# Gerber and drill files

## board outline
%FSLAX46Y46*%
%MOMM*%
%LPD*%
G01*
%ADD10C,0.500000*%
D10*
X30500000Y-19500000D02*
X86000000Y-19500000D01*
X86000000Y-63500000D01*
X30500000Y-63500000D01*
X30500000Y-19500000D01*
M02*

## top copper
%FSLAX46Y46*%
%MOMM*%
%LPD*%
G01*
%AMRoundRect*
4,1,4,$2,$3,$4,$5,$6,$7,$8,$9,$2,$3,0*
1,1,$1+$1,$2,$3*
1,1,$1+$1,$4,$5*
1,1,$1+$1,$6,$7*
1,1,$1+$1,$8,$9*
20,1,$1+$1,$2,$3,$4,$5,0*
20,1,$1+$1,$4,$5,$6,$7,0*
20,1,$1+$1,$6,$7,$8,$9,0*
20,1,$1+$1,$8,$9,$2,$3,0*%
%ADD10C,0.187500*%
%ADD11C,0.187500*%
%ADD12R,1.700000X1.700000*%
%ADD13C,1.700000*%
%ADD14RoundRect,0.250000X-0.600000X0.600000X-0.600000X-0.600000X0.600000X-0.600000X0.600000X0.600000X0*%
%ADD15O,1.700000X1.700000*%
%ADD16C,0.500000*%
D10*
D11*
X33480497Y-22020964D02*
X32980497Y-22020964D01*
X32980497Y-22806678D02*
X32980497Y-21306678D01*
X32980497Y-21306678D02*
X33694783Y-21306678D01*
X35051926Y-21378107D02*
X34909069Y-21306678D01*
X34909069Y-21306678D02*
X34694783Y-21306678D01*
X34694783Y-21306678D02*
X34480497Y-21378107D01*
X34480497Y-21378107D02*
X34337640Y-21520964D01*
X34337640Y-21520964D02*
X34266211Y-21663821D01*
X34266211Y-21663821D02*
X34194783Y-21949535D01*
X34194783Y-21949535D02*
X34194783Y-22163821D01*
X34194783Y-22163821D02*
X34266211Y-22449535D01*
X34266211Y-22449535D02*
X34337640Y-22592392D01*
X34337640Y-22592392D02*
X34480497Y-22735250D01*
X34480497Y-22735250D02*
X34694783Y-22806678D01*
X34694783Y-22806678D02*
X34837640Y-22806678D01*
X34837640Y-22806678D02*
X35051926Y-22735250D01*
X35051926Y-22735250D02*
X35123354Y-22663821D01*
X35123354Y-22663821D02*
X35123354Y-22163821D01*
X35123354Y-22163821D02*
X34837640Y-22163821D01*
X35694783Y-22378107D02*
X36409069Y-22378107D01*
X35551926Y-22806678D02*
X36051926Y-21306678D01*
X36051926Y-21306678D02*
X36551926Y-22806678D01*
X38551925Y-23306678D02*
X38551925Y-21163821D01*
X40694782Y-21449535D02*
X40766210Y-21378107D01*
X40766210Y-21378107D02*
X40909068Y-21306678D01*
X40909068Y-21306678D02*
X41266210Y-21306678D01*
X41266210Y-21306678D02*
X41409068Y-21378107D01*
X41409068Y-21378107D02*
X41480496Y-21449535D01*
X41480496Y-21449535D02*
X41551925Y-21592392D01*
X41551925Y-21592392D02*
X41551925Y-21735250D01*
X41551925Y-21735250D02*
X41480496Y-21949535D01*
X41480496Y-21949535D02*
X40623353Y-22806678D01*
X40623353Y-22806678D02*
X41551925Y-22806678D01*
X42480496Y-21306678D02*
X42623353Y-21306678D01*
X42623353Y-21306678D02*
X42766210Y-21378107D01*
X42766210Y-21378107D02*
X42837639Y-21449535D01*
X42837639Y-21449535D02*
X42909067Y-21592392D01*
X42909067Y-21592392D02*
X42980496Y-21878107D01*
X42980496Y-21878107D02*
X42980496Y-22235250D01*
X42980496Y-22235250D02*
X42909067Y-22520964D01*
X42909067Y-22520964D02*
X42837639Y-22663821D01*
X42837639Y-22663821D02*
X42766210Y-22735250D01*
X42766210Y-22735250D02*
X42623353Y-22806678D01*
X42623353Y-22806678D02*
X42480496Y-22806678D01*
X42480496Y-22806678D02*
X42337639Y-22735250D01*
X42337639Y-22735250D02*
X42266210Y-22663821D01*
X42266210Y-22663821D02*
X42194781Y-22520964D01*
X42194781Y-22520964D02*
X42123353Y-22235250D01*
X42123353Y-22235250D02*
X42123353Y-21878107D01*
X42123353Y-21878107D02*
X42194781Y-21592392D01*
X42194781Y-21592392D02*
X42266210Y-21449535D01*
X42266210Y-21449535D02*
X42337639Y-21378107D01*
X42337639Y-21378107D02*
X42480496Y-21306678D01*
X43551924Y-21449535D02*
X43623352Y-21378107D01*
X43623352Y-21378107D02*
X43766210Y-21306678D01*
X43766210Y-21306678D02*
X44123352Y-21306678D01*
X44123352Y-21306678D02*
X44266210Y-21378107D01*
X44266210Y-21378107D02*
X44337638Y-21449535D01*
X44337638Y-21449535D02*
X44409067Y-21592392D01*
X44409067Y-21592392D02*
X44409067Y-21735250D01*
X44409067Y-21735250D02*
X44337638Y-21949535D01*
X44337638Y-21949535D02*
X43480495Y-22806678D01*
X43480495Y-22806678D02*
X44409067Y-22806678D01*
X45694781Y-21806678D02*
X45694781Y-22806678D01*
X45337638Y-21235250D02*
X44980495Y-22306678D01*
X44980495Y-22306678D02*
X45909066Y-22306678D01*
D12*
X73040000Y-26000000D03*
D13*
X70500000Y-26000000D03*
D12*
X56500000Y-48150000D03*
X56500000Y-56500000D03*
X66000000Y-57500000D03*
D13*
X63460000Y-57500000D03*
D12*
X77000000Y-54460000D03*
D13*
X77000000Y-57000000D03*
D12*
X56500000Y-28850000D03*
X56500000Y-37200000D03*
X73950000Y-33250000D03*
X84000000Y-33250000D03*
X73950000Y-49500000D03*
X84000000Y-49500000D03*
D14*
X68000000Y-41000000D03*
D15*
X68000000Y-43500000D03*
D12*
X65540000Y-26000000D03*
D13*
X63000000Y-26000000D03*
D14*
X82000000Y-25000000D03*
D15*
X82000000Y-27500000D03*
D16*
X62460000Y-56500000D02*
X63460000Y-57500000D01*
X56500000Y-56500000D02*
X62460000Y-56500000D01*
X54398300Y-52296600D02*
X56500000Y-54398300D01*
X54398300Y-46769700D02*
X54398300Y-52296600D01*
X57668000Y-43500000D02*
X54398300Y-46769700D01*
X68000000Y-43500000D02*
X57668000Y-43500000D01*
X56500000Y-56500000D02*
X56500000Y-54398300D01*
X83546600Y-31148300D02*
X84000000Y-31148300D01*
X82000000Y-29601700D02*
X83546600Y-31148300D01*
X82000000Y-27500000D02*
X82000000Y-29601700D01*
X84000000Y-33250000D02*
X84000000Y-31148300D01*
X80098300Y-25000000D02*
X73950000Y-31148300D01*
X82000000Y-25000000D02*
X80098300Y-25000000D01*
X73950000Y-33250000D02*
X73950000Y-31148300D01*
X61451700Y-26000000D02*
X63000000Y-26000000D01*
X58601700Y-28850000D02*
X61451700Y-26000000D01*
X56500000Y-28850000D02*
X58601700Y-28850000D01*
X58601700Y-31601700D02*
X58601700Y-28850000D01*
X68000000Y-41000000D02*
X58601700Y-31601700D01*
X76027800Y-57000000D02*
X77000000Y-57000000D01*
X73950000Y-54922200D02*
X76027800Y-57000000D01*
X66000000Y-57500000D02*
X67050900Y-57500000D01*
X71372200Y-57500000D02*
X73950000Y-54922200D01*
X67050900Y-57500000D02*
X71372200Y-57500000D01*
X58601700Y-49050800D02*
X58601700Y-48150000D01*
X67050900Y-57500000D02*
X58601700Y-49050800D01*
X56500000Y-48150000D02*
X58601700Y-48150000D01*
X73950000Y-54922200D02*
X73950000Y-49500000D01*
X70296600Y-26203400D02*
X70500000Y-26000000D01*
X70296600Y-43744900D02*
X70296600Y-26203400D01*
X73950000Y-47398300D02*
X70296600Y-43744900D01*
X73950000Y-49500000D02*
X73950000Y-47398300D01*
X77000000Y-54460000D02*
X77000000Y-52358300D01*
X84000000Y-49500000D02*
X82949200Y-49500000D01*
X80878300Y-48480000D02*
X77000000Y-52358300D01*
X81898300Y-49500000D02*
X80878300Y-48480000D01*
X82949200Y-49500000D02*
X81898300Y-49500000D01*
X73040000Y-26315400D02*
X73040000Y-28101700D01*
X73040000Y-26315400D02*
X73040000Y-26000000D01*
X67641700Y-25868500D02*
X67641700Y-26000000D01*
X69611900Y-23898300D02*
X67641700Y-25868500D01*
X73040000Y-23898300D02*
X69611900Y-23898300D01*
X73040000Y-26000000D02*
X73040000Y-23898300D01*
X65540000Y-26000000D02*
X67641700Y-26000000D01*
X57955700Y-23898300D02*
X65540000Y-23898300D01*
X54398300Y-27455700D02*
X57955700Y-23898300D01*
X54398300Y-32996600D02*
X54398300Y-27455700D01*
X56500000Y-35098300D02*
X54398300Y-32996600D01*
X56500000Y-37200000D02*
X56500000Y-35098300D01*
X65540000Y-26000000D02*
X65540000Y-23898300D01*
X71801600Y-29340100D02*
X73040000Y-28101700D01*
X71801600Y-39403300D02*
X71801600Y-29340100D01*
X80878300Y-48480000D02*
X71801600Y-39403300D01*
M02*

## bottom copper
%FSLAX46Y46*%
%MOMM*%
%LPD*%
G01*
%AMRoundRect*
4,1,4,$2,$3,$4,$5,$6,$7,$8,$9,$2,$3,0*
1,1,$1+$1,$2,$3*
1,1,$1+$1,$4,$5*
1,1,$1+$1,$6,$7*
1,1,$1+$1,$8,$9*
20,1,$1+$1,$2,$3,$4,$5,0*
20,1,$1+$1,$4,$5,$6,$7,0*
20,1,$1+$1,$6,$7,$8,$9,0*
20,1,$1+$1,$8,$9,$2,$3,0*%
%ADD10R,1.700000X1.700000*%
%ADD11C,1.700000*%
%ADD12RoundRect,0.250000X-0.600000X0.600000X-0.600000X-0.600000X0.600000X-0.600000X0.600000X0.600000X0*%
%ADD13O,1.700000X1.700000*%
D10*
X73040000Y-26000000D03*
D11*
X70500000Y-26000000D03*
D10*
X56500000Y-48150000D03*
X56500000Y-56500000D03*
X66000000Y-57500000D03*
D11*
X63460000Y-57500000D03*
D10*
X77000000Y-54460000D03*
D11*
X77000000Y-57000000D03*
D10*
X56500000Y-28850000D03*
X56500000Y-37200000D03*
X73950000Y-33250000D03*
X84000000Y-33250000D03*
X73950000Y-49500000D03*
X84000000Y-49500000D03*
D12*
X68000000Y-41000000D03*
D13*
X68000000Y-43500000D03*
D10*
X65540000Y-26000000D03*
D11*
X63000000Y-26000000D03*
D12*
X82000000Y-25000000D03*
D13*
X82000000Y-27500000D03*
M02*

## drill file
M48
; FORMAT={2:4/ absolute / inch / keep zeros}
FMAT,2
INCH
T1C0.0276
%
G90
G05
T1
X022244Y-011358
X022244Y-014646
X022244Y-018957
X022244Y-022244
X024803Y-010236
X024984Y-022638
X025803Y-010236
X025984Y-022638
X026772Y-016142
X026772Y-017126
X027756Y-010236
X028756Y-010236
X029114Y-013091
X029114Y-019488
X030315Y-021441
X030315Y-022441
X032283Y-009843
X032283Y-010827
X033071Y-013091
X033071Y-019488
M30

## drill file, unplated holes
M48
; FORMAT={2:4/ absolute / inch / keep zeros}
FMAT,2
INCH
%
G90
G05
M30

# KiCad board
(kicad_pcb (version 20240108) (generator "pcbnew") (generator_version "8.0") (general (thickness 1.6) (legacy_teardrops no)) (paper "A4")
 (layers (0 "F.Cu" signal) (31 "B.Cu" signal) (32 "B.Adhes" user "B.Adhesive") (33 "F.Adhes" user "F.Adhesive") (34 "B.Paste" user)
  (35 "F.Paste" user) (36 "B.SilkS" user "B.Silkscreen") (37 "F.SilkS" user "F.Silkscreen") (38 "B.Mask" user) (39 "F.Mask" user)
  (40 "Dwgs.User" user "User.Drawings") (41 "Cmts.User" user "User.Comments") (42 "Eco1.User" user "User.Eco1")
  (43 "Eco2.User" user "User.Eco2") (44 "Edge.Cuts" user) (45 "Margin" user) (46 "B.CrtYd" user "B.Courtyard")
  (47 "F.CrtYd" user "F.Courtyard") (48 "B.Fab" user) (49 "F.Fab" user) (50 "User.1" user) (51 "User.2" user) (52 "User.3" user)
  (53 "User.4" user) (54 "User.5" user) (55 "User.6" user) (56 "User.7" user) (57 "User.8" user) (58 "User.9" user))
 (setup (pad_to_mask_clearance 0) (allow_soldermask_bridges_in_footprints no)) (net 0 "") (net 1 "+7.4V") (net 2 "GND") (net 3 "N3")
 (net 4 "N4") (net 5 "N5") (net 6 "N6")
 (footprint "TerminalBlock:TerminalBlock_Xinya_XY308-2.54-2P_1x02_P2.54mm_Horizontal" (layer "F.Cu") (at 73.04 26 180)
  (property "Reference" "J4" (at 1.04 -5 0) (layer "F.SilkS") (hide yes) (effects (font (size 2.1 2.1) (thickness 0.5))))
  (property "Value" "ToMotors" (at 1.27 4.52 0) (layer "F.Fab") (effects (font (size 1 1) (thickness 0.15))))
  (pad "1" thru_hole rect (at 0 0 180) (size 1.7 1.7) (drill 0.7) (layers "*.Cu" "*.Mask") (remove_unused_layers no) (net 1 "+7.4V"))
  (pad "2" thru_hole circle (at 2.54 0 180) (size 1.7 1.7) (drill 0.7) (layers "*.Cu" "*.Mask") (remove_unused_layers no) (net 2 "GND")))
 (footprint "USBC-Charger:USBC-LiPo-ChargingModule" (layer "F.Cu") (at 45.5 61.6)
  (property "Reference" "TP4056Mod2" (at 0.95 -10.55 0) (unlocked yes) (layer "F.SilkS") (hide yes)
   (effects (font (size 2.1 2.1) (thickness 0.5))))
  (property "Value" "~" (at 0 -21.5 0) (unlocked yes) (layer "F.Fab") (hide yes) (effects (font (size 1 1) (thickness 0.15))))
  (pad "1" thru_hole rect (at 11 -13.45) (size 1.7 1.7) (drill 0.7) (layers "*.Cu" "*.Mask") (remove_unused_layers no) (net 2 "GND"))
  (pad "2" thru_hole rect (at 11 -5.1) (size 1.7 1.7) (drill 0.7) (layers "*.Cu" "*.Mask") (remove_unused_layers no) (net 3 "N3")))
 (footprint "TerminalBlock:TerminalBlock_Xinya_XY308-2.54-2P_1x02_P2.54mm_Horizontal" (layer "F.Cu") (at 66 57.5 180)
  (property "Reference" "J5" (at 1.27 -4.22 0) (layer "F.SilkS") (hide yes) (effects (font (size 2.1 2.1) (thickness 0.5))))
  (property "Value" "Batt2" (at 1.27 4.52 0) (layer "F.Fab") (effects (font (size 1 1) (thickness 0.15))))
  (pad "1" thru_hole rect (at 0 0 180) (size 1.7 1.7) (drill 0.7) (layers "*.Cu" "*.Mask") (remove_unused_layers no) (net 2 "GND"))
  (pad "2" thru_hole circle (at 2.54 0 180) (size 1.7 1.7) (drill 0.7) (layers "*.Cu" "*.Mask") (remove_unused_layers no) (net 3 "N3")))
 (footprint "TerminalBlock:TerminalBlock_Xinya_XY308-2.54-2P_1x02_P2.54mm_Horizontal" (layer "F.Cu") (at 77 54.46 -90)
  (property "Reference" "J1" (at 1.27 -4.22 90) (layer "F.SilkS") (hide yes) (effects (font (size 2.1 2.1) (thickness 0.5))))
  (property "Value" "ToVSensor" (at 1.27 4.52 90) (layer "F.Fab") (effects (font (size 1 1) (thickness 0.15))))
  (pad "1" thru_hole rect (at 0 0 270) (size 1.7 1.7) (drill 0.7) (layers "*.Cu" "*.Mask") (remove_unused_layers no) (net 1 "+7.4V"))
  (pad "2" thru_hole circle (at 2.54 0 270) (size 1.7 1.7) (drill 0.7) (layers "*.Cu" "*.Mask") (remove_unused_layers no) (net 2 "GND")))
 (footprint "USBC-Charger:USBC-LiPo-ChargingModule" (layer "F.Cu") (at 45.5 42.3)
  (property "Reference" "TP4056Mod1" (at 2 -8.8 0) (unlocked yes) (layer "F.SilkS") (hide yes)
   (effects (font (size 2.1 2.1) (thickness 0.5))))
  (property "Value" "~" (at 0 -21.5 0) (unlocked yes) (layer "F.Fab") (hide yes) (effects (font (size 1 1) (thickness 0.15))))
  (pad "1" thru_hole rect (at 11 -13.45) (size 1.7 1.7) (drill 0.7) (layers "*.Cu" "*.Mask") (remove_unused_layers no) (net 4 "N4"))
  (pad "2" thru_hole rect (at 11 -5.1) (size 1.7 1.7) (drill 0.7) (layers "*.Cu" "*.Mask") (remove_unused_layers no) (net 1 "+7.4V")))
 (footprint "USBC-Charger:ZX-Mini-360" (layer "F.Cu") (at 84.95 50.5 90)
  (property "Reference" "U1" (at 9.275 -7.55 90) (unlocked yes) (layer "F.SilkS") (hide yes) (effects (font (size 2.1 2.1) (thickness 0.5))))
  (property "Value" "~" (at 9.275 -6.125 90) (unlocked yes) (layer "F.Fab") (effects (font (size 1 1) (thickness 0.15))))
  (pad "1" thru_hole rect (at 17.25 -11 90) (size 1.7 1.7) (drill 0.7) (layers "*.Cu" "*.Mask") (remove_unused_layers no) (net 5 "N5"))
  (pad "2" thru_hole rect (at 17.25 -0.95 90) (size 1.7 1.7) (drill 0.7) (layers "*.Cu" "*.Mask") (remove_unused_layers no) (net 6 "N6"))
  (pad "3" thru_hole rect (at 1 -11 90) (size 1.7 1.7) (drill 0.7) (layers "*.Cu" "*.Mask") (remove_unused_layers no) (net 2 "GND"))
  (pad "4" thru_hole rect (at 1 -0.95 90) (size 1.7 1.7) (drill 0.7) (layers "*.Cu" "*.Mask") (remove_unused_layers no) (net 1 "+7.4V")))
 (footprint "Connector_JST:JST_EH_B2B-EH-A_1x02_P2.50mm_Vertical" (layer "F.Cu") (at 68 41 -90)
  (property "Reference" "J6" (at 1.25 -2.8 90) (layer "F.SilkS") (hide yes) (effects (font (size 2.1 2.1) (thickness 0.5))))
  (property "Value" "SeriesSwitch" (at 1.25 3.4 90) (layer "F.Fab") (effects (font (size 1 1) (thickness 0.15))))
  (pad "1" thru_hole roundrect (at 0 0 270) (size 1.7 1.7) (drill 0.7) (layers "*.Cu" "*.Mask") (remove_unused_layers no)
   (roundrect_rratio 0.147059) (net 4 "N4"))
  (pad "2" thru_hole oval (at 2.5 0 270) (size 1.7 1.7) (drill 0.7) (layers "*.Cu" "*.Mask") (remove_unused_layers no) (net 3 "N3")))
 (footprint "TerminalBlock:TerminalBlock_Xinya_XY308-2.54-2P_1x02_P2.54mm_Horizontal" (layer "F.Cu") (at 65.54 26 180)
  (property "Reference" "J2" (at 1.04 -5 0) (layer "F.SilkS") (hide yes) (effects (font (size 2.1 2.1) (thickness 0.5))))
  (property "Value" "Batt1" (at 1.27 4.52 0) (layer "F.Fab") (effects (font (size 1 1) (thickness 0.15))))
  (pad "1" thru_hole rect (at 0 0 180) (size 1.7 1.7) (drill 0.7) (layers "*.Cu" "*.Mask") (remove_unused_layers no) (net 1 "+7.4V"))
  (pad "2" thru_hole circle (at 2.54 0 180) (size 1.7 1.7) (drill 0.7) (layers "*.Cu" "*.Mask") (remove_unused_layers no) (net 4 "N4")))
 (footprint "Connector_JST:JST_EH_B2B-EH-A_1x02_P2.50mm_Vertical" (layer "F.Cu") (at 82 25 -90)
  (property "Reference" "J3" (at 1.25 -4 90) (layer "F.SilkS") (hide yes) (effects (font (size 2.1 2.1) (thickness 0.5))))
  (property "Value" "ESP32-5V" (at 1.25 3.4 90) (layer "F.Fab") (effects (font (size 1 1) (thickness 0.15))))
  (pad "1" thru_hole roundrect (at 0 0 270) (size 1.7 1.7) (drill 0.7) (layers "*.Cu" "*.Mask") (remove_unused_layers no)
   (roundrect_rratio 0.147059) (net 5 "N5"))
  (pad "2" thru_hole oval (at 2.5 0 270) (size 1.7 1.7) (drill 0.7) (layers "*.Cu" "*.Mask") (remove_unused_layers no) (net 6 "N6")))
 (gr_rect (start 30.5 19.5) (end 86 63.5) (stroke (width 0.5) (type default)) (fill none) (layer "Edge.Cuts"))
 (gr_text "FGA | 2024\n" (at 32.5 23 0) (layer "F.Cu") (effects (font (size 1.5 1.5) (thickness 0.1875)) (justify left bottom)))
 (segment (start 69.6119 23.8983) (end 67.6417 25.8685) (width 0.5) (layer "F.Cu") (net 1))
 (segment (start 80.8783 48.48) (end 71.8016 39.4033) (width 0.5) (layer "F.Cu") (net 1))
 (segment (start 82.9492 49.5) (end 81.8983 49.5) (width 0.5) (layer "F.Cu") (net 1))
 (segment (start 77 54.46) (end 77 52.3583) (width 0.5) (layer "F.Cu") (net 1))
 (segment (start 57.9557 23.8983) (end 65.54 23.8983) (width 0.5) (layer "F.Cu") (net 1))
 (segment (start 54.3983 32.9966) (end 54.3983 27.4557) (width 0.5) (layer "F.Cu") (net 1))
 (segment (start 56.5 37.2) (end 56.5 35.0983) (width 0.5) (layer "F.Cu") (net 1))
 (segment (start 56.5 35.0983) (end 54.3983 32.9966) (width 0.5) (layer "F.Cu") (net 1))
 (segment (start 73.04 23.8983) (end 69.6119 23.8983) (width 0.5) (layer "F.Cu") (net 1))
 (segment (start 81.8983 49.5) (end 80.8783 48.48) (width 0.5) (layer "F.Cu") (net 1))
 (segment (start 65.54 26) (end 65.54 23.8983) (width 0.5) (layer "F.Cu") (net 1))
 (segment (start 80.8783 48.48) (end 77 52.3583) (width 0.5) (layer "F.Cu") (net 1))
 (segment (start 54.3983 27.4557) (end 57.9557 23.8983) (width 0.5) (layer "F.Cu") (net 1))
 (segment (start 67.6417 25.8685) (end 67.6417 26) (width 0.5) (layer "F.Cu") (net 1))
 (segment (start 73.04 26.3154) (end 73.04 28.1017) (width 0.5) (layer "F.Cu") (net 1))
 (segment (start 71.8016 29.3401) (end 73.04 28.1017) (width 0.5) (layer "F.Cu") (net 1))
 (segment (start 84 49.5) (end 82.9492 49.5) (width 0.5) (layer "F.Cu") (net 1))
 (segment (start 73.04 26) (end 73.04 23.8983) (width 0.5) (layer "F.Cu") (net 1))
 (segment (start 73.04 26.3154) (end 73.04 26) (width 0.5) (layer "F.Cu") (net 1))
 (segment (start 65.54 26) (end 67.6417 26) (width 0.5) (layer "F.Cu") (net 1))
 (segment (start 71.8016 39.4033) (end 71.8016 29.3401) (width 0.5) (layer "F.Cu") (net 1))
 (segment (start 56.5 48.15) (end 58.6017 48.15) (width 0.5) (layer "F.Cu") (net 2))
 (segment (start 73.95 49.5) (end 73.95 47.3983) (width 0.5) (layer "F.Cu") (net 2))
 (segment (start 70.2966 26.2034) (end 70.5 26) (width 0.5) (layer "F.Cu") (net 2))
 (segment (start 73.95 54.9222) (end 73.95 49.5) (width 0.5) (layer "F.Cu") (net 2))
 (segment (start 66 57.5) (end 67.0509 57.5) (width 0.5) (layer "F.Cu") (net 2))
 (segment (start 73.95 54.9222) (end 76.0278 57) (width 0.5) (layer "F.Cu") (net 2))
 (segment (start 73.95 47.3983) (end 70.2966 43.7449) (width 0.5) (layer "F.Cu") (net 2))
 (segment (start 70.2966 43.7449) (end 70.2966 26.2034) (width 0.5) (layer "F.Cu") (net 2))
 (segment (start 58.6017 49.0508) (end 58.6017 48.15) (width 0.5) (layer "F.Cu") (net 2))
 (segment (start 67.0509 57.5) (end 71.3722 57.5) (width 0.5) (layer "F.Cu") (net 2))
 (segment (start 76.0278 57) (end 77 57) (width 0.5) (layer "F.Cu") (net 2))
 (segment (start 71.3722 57.5) (end 73.95 54.9222) (width 0.5) (layer "F.Cu") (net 2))
 (segment (start 67.0509 57.5) (end 58.6017 49.0508) (width 0.5) (layer "F.Cu") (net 2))
 (segment (start 68 41) (end 58.6017 31.6017) (width 0.5) (layer "F.Cu") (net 4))
 (segment (start 61.4517 26) (end 63 26) (width 0.5) (layer "F.Cu") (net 4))
 (segment (start 56.5 28.85) (end 58.6017 28.85) (width 0.5) (layer "F.Cu") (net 4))
 (segment (start 58.6017 31.6017) (end 58.6017 28.85) (width 0.5) (layer "F.Cu") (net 4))
 (segment (start 58.6017 28.85) (end 61.4517 26) (width 0.5) (layer "F.Cu") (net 4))
 (segment (start 82 25) (end 80.0983 25) (width 0.5) (layer "F.Cu") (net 5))
 (segment (start 80.0983 25) (end 73.95 31.1483) (width 0.5) (layer "F.Cu") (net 5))
 (segment (start 73.95 33.25) (end 73.95 31.1483) (width 0.5) (layer "F.Cu") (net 5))
 (segment (start 84 33.25) (end 84 31.1483) (width 0.5) (layer "F.Cu") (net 6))
 (segment (start 82 29.6017) (end 83.5466 31.1483) (width 0.5) (layer "F.Cu") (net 6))
 (segment (start 82 27.5) (end 82 29.6017) (width 0.5) (layer "F.Cu") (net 6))
 (segment (start 83.5466 31.1483) (end 84 31.1483) (width 0.5) (layer "F.Cu") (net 6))
 (segment (start 54.3983 52.2966) (end 56.5 54.3983) (width 0.5) (layer "F.Cu") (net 3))
 (segment (start 62.46 56.5) (end 63.46 57.5) (width 0.5) (layer "F.Cu") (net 3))
 (segment (start 56.5 56.5) (end 56.5 54.3983) (width 0.5) (layer "F.Cu") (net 3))
 (segment (start 68 43.5) (end 57.668 43.5) (width 0.5) (layer "F.Cu") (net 3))
 (segment (start 54.3983 46.7697) (end 54.3983 52.2966) (width 0.5) (layer "F.Cu") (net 3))
 (segment (start 56.5 56.5) (end 62.46 56.5) (width 0.5) (layer "F.Cu") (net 3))
 (segment (start 57.668 43.5) (end 54.3983 46.7697) (width 0.5) (layer "F.Cu") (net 3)))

